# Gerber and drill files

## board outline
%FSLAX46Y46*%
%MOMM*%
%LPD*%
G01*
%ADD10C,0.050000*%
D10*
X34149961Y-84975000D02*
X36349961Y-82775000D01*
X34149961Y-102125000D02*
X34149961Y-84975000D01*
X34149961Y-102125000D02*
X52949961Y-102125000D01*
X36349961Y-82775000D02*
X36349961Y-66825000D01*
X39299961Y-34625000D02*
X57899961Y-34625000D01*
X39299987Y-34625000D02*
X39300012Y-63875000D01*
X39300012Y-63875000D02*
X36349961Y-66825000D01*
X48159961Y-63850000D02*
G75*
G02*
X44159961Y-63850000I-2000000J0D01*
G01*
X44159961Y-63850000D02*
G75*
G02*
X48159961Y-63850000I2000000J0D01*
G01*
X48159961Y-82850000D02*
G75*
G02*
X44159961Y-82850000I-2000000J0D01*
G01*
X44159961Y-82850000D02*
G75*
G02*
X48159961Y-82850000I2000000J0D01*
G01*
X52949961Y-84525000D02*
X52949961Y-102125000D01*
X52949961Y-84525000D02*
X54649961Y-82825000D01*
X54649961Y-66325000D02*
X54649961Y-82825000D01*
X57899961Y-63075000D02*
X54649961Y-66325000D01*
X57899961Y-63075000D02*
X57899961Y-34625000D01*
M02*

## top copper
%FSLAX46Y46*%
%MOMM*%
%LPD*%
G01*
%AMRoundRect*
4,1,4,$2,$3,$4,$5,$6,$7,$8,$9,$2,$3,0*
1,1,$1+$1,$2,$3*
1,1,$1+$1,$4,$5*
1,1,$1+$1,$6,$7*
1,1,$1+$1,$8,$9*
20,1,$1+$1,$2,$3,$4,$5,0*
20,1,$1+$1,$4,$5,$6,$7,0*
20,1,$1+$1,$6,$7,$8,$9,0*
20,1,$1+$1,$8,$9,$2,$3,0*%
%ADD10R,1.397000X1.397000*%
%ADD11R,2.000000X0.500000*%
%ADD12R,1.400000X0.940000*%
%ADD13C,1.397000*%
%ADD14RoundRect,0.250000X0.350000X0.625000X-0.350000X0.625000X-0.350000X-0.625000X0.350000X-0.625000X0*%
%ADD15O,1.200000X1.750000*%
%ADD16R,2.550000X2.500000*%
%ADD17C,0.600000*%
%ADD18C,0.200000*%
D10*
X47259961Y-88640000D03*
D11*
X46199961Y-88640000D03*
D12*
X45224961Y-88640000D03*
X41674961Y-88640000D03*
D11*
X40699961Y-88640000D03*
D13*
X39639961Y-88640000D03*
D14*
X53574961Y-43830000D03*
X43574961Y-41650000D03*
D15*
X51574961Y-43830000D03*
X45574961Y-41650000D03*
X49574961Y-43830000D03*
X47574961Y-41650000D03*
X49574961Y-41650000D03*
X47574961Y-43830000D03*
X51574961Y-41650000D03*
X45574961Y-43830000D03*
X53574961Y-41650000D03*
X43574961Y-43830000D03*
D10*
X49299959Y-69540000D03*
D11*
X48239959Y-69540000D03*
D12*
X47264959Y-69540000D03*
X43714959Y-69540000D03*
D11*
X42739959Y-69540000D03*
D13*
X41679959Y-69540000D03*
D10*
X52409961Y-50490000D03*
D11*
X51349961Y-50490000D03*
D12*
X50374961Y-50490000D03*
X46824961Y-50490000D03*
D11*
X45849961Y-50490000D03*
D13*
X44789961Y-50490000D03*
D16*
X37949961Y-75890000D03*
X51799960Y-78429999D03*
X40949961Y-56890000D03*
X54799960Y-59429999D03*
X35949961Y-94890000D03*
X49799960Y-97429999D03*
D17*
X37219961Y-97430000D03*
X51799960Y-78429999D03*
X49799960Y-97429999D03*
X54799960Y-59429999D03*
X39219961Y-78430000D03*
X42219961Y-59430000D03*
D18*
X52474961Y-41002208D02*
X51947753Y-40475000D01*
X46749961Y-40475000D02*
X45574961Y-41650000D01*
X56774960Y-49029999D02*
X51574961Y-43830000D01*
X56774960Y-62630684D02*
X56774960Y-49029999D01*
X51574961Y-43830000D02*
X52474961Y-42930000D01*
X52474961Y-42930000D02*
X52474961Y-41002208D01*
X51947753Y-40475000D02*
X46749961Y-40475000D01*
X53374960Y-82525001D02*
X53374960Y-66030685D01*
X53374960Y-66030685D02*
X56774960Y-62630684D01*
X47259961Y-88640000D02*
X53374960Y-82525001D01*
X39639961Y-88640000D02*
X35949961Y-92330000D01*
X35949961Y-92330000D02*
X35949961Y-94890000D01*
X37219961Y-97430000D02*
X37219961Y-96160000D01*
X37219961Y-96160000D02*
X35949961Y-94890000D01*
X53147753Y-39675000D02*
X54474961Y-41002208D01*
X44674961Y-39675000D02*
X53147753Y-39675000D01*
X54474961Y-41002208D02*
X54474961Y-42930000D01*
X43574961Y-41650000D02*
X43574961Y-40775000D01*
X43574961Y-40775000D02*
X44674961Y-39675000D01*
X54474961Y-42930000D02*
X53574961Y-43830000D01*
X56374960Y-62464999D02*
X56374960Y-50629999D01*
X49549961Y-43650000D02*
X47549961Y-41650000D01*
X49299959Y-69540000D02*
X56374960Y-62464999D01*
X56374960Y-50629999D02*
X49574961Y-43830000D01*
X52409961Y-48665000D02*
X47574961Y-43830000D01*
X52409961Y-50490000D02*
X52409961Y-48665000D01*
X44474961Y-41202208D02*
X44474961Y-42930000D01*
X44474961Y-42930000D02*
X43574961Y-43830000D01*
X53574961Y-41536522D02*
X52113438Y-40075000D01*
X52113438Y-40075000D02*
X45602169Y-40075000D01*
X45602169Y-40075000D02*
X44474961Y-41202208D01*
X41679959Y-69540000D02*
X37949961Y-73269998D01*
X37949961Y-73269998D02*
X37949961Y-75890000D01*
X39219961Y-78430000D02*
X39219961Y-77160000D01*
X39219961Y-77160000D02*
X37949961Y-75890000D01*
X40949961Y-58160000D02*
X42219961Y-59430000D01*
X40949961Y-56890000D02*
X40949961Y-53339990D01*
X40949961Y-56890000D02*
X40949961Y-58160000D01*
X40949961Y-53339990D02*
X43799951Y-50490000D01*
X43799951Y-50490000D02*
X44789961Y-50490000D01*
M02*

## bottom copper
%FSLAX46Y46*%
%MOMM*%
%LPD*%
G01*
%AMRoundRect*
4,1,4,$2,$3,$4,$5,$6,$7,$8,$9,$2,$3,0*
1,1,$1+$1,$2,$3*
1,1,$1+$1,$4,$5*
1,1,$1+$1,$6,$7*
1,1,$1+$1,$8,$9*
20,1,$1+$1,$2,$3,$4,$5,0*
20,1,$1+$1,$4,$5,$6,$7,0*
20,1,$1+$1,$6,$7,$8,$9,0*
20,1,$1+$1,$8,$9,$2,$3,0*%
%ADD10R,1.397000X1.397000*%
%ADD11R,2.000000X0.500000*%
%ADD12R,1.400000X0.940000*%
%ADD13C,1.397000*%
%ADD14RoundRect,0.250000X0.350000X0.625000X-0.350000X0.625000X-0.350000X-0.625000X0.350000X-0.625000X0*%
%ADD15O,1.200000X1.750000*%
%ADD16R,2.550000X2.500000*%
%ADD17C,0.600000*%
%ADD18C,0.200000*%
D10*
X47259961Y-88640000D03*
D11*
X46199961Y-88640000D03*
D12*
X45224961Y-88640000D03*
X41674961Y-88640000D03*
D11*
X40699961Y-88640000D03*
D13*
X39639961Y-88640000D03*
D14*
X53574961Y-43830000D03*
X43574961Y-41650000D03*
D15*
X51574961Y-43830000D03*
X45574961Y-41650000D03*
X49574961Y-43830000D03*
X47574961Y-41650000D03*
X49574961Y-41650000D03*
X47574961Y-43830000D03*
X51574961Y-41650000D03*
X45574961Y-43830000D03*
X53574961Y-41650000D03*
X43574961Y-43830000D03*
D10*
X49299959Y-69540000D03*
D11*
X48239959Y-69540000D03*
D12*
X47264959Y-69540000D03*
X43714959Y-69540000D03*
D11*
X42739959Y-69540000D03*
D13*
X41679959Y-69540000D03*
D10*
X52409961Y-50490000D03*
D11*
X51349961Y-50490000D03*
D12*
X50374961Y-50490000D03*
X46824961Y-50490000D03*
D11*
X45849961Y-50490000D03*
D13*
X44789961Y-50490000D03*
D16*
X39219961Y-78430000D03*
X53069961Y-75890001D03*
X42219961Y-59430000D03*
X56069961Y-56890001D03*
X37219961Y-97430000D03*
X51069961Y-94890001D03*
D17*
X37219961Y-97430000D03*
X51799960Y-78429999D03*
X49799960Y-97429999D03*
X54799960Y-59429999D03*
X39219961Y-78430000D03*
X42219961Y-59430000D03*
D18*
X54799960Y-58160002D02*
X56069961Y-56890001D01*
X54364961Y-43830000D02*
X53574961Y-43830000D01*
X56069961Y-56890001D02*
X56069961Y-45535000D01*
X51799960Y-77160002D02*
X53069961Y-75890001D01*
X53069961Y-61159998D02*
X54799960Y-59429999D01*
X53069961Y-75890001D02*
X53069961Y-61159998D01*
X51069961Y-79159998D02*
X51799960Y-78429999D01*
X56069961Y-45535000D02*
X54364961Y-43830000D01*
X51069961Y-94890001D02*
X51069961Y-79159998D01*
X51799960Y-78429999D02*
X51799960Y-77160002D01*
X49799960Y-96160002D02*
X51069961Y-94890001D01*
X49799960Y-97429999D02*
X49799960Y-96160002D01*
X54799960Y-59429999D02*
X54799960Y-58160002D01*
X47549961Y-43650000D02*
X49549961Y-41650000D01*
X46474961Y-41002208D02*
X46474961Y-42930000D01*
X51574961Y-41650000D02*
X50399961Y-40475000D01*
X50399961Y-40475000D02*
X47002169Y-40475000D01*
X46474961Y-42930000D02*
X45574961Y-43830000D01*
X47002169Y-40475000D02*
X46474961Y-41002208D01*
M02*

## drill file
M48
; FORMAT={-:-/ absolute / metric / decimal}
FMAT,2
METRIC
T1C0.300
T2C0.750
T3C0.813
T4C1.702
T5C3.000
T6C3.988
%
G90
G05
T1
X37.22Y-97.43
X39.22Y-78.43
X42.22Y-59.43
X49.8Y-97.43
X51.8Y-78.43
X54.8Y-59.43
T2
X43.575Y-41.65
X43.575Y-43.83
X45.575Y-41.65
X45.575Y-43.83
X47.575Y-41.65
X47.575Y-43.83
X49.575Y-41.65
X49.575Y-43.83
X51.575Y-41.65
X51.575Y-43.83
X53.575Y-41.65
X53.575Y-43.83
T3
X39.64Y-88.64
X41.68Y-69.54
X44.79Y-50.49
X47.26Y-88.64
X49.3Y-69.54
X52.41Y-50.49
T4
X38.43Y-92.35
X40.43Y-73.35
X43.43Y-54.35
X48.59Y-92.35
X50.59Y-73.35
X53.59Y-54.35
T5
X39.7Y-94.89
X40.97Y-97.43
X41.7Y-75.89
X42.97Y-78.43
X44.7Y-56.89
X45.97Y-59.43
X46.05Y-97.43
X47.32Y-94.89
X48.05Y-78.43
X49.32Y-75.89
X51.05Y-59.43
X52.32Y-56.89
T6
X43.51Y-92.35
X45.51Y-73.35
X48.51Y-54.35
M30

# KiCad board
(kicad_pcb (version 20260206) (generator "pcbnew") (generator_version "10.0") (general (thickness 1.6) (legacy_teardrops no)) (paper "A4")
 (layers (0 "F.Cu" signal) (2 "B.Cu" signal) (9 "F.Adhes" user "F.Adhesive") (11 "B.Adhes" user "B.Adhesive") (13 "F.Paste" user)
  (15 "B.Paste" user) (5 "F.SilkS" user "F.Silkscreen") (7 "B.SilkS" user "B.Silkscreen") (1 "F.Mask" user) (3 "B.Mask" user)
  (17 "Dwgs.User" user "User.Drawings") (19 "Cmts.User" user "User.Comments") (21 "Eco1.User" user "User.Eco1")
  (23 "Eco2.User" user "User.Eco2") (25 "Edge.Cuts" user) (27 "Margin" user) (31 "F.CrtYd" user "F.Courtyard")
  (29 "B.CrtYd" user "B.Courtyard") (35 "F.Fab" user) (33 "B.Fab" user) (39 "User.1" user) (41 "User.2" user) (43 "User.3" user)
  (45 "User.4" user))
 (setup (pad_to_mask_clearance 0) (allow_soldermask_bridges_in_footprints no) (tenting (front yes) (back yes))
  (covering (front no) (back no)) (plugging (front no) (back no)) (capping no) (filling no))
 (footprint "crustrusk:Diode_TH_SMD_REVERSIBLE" (layer "F.Cu") (at 43.449961 88.64 180)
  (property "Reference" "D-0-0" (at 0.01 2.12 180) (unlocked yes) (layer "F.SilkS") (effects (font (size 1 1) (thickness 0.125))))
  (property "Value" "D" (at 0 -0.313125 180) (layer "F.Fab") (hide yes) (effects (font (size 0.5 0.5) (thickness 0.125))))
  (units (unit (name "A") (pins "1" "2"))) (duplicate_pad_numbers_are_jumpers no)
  (pad "1" thru_hole rect (at -3.81 0 180) (size 1.397 1.397) (drill 0.8128) (layers "*.Cu" "*.Mask") (remove_unused_layers no)
   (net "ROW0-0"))
  (pad "1" smd rect (at -2.75 0) (size 2 0.5) (layers "F.Cu") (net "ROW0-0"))
  (pad "1" smd rect (at -2.75 0 180) (size 2 0.5) (layers "B.Cu") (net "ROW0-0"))
  (pad "1" smd rect (at -1.775 0) (size 1.4 0.94) (layers "F.Cu" "F.Mask" "F.Paste") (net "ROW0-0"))
  (pad "1" smd rect (at -1.775 0 180) (size 1.4 0.94) (layers "B.Cu" "B.Mask" "B.Paste") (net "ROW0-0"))
  (pad "2" smd rect (at 1.775 0) (size 1.4 0.94) (layers "F.Cu" "F.Mask" "F.Paste") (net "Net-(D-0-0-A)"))
  (pad "2" smd rect (at 1.775 0 180) (size 1.4 0.94) (layers "B.Cu" "B.Mask" "B.Paste") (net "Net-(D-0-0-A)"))
  (pad "2" smd rect (at 2.75 0) (size 2 0.5) (layers "F.Cu") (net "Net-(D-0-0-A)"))
  (pad "2" smd rect (at 2.75 0 180) (size 2 0.5) (layers "B.Cu") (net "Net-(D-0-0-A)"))
  (pad "2" thru_hole circle (at 3.81 0 180) (size 1.397 1.397) (drill 0.8128) (layers "*.Cu" "*.Mask") (remove_unused_layers no)
   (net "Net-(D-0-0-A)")))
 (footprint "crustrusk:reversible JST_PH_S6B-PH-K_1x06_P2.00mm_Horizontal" (layer "F.Cu") (at 53.574961 43.83 180)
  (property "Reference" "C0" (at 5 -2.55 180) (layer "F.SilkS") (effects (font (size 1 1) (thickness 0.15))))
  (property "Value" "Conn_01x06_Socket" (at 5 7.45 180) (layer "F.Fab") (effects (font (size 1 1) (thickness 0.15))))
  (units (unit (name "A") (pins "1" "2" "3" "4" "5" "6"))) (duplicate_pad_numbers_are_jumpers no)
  (pad "1" thru_hole roundrect (at 0 0 180) (size 1.2 1.75) (drill 0.75) (layers "*.Cu" "*.Mask") (remove_unused_layers no)
   (roundrect_rratio 0.208333) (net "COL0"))
  (pad "1" thru_hole roundrect (at 10 2.18 180) (size 1.2 1.75) (drill 0.75) (layers "*.Cu" "*.Mask") (remove_unused_layers no)
   (roundrect_rratio 0.208333) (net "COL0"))
  (pad "2" thru_hole oval (at 2 0 180) (size 1.2 1.75) (drill 0.75) (layers "*.Cu" "*.Mask") (remove_unused_layers no) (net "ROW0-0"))
  (pad "2" thru_hole oval (at 8 2.18 180) (size 1.2 1.75) (drill 0.75) (layers "*.Cu" "*.Mask") (remove_unused_layers no) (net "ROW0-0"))
  (pad "3" thru_hole oval (at 4 0 180) (size 1.2 1.75) (drill 0.75) (layers "*.Cu" "*.Mask") (remove_unused_layers no) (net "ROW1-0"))
  (pad "3" thru_hole oval (at 6 2.18 180) (size 1.2 1.75) (drill 0.75) (layers "*.Cu" "*.Mask") (remove_unused_layers no) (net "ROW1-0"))
  (pad "4" thru_hole oval (at 4 2.18 180) (size 1.2 1.75) (drill 0.75) (layers "*.Cu" "*.Mask") (remove_unused_layers no) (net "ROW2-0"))
  (pad "4" thru_hole oval (at 6 0 180) (size 1.2 1.75) (drill 0.75) (layers "*.Cu" "*.Mask") (remove_unused_layers no) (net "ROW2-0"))
  (pad "5" thru_hole oval (at 2 2.18 180) (size 1.2 1.75) (drill 0.75) (layers "*.Cu" "*.Mask") (remove_unused_layers no) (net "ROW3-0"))
  (pad "5" thru_hole oval (at 8 0 180) (size 1.2 1.75) (drill 0.75) (layers "*.Cu" "*.Mask") (remove_unused_layers no) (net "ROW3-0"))
  (pad "6" thru_hole oval (at 0 2.18 180) (size 1.2 1.75) (drill 0.75) (layers "*.Cu" "*.Mask") (remove_unused_layers no) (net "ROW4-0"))
  (pad "6" thru_hole oval (at 10 0 180) (size 1.2 1.75) (drill 0.75) (layers "*.Cu" "*.Mask") (remove_unused_layers no) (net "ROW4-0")))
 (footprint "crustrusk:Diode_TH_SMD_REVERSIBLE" (layer "F.Cu") (at 45.489959 69.54 180)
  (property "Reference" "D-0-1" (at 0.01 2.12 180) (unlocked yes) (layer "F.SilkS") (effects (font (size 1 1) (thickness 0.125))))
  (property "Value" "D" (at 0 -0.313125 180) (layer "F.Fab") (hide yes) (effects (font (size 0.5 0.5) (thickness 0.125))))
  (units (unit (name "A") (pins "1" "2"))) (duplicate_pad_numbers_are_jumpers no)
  (pad "1" thru_hole rect (at -3.81 0 180) (size 1.397 1.397) (drill 0.8128) (layers "*.Cu" "*.Mask") (remove_unused_layers no)
   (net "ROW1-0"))
  (pad "1" smd rect (at -2.75 0) (size 2 0.5) (layers "F.Cu") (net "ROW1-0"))
  (pad "1" smd rect (at -2.75 0 180) (size 2 0.5) (layers "B.Cu") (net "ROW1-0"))
  (pad "1" smd rect (at -1.775 0) (size 1.4 0.94) (layers "F.Cu" "F.Mask" "F.Paste") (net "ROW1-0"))
  (pad "1" smd rect (at -1.775 0 180) (size 1.4 0.94) (layers "B.Cu" "B.Mask" "B.Paste") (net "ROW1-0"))
  (pad "2" smd rect (at 1.775 0) (size 1.4 0.94) (layers "F.Cu" "F.Mask" "F.Paste") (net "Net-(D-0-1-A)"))
  (pad "2" smd rect (at 1.775 0 180) (size 1.4 0.94) (layers "B.Cu" "B.Mask" "B.Paste") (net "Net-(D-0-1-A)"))
  (pad "2" smd rect (at 2.75 0) (size 2 0.5) (layers "F.Cu") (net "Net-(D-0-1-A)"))
  (pad "2" smd rect (at 2.75 0 180) (size 2 0.5) (layers "B.Cu") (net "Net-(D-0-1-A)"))
  (pad "2" thru_hole circle (at 3.81 0 180) (size 1.397 1.397) (drill 0.8128) (layers "*.Cu" "*.Mask") (remove_unused_layers no)
   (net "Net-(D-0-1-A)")))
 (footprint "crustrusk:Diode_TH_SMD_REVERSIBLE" (layer "F.Cu") (at 48.599961 50.49 180)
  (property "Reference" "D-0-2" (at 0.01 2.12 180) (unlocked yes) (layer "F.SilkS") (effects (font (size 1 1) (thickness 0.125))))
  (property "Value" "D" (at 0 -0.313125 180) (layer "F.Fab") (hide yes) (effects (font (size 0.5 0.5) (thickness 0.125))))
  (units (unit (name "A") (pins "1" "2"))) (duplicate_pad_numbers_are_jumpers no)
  (pad "1" thru_hole rect (at -3.81 0 180) (size 1.397 1.397) (drill 0.8128) (layers "*.Cu" "*.Mask") (remove_unused_layers no)
   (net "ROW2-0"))
  (pad "1" smd rect (at -2.75 0) (size 2 0.5) (layers "F.Cu") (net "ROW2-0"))
  (pad "1" smd rect (at -2.75 0 180) (size 2 0.5) (layers "B.Cu") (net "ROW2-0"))
  (pad "1" smd rect (at -1.775 0) (size 1.4 0.94) (layers "F.Cu" "F.Mask" "F.Paste") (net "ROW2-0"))
  (pad "1" smd rect (at -1.775 0 180) (size 1.4 0.94) (layers "B.Cu" "B.Mask" "B.Paste") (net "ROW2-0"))
  (pad "2" smd rect (at 1.775 0) (size 1.4 0.94) (layers "F.Cu" "F.Mask" "F.Paste") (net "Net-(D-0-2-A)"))
  (pad "2" smd rect (at 1.775 0 180) (size 1.4 0.94) (layers "B.Cu" "B.Mask" "B.Paste") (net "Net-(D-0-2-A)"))
  (pad "2" smd rect (at 2.75 0) (size 2 0.5) (layers "F.Cu") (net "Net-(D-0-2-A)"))
  (pad "2" smd rect (at 2.75 0 180) (size 2 0.5) (layers "B.Cu") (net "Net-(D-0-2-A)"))
  (pad "2" thru_hole circle (at 3.81 0 180) (size 1.397 1.397) (drill 0.8128) (layers "*.Cu" "*.Mask") (remove_unused_layers no)
   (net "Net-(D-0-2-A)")))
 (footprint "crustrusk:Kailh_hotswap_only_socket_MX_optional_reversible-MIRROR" (layer "F.Cu") (at 45.509961 73.35 180)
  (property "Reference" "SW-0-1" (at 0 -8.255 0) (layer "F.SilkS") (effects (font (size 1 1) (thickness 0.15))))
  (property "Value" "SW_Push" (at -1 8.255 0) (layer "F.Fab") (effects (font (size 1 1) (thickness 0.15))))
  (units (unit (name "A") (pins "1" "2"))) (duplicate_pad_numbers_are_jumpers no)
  (pad "" np_thru_hole circle (at -5.08 0 180) (size 1.7018 1.7018) (drill 1.7018) (layers "*.Cu" "*.Mask"))
  (pad "" np_thru_hole circle (at -3.81 -2.54) (size 3 3) (drill 3) (layers "*.Cu" "*.Mask"))
  (pad "" np_thru_hole circle (at -2.54 -5.079998 180) (size 3 3) (drill 3) (layers "*.Cu" "*.Mask"))
  (pad "" np_thru_hole circle (at 0 0 180) (size 3.9878 3.9878) (drill 3.9878) (layers "*.Cu" "*.Mask"))
  (pad "" np_thru_hole circle (at 2.540002 -5.080001) (size 3 3) (drill 3) (layers "*.Cu" "*.Mask"))
  (pad "" np_thru_hole circle (at 3.81 -2.54 180) (size 3 3) (drill 3) (layers "*.Cu" "*.Mask"))
  (pad "" np_thru_hole circle (at 5.08 0 180) (size 1.7018 1.7018) (drill 1.7018) (layers "*.Cu" "*.Mask"))
  (pad "1" smd rect (at 6.29 -5.08) (size 2.55 2.5) (layers "B.Cu" "B.Mask" "B.Paste") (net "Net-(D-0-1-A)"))
  (pad "1" smd rect (at 7.56 -2.54 180) (size 2.55 2.5) (layers "F.Cu" "F.Mask" "F.Paste") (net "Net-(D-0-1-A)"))
  (pad "2" smd rect (at -7.56 -2.540001) (size 2.55 2.5) (layers "B.Cu" "B.Mask" "B.Paste") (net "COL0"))
  (pad "2" smd rect (at -6.289999 -5.079999 180) (size 2.55 2.5) (layers "F.Cu" "F.Mask" "F.Paste") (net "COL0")))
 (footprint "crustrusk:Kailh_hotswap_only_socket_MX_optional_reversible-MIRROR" (layer "F.Cu") (at 48.509961 54.35 180)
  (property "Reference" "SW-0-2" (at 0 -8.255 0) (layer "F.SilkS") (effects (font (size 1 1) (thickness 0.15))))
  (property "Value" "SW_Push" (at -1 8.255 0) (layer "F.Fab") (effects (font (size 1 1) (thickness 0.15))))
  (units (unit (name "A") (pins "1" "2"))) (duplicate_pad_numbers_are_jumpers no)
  (pad "" np_thru_hole circle (at -5.08 0 180) (size 1.7018 1.7018) (drill 1.7018) (layers "*.Cu" "*.Mask"))
  (pad "" np_thru_hole circle (at -3.81 -2.54) (size 3 3) (drill 3) (layers "*.Cu" "*.Mask"))
  (pad "" np_thru_hole circle (at -2.54 -5.079998 180) (size 3 3) (drill 3) (layers "*.Cu" "*.Mask"))
  (pad "" np_thru_hole circle (at 0 0 180) (size 3.9878 3.9878) (drill 3.9878) (layers "*.Cu" "*.Mask"))
  (pad "" np_thru_hole circle (at 2.540002 -5.080001) (size 3 3) (drill 3) (layers "*.Cu" "*.Mask"))
  (pad "" np_thru_hole circle (at 3.81 -2.54 180) (size 3 3) (drill 3) (layers "*.Cu" "*.Mask"))
  (pad "" np_thru_hole circle (at 5.08 0 180) (size 1.7018 1.7018) (drill 1.7018) (layers "*.Cu" "*.Mask"))
  (pad "1" smd rect (at 6.29 -5.08) (size 2.55 2.5) (layers "B.Cu" "B.Mask" "B.Paste") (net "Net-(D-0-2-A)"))
  (pad "1" smd rect (at 7.56 -2.54 180) (size 2.55 2.5) (layers "F.Cu" "F.Mask" "F.Paste") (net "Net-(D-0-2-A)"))
  (pad "2" smd rect (at -7.56 -2.540001) (size 2.55 2.5) (layers "B.Cu" "B.Mask" "B.Paste") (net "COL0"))
  (pad "2" smd rect (at -6.289999 -5.079999 180) (size 2.55 2.5) (layers "F.Cu" "F.Mask" "F.Paste") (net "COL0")))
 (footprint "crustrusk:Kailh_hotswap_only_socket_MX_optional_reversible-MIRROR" (layer "F.Cu") (at 43.509961 92.35 180)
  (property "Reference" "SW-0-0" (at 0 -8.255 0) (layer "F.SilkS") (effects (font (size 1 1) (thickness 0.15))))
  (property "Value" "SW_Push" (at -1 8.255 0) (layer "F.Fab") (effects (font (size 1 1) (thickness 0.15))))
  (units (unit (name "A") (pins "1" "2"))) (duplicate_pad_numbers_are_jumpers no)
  (pad "" np_thru_hole circle (at -5.08 0 180) (size 1.7018 1.7018) (drill 1.7018) (layers "*.Cu" "*.Mask"))
  (pad "" np_thru_hole circle (at -3.81 -2.54) (size 3 3) (drill 3) (layers "*.Cu" "*.Mask"))
  (pad "" np_thru_hole circle (at -2.54 -5.079998 180) (size 3 3) (drill 3) (layers "*.Cu" "*.Mask"))
  (pad "" np_thru_hole circle (at 0 0 180) (size 3.9878 3.9878) (drill 3.9878) (layers "*.Cu" "*.Mask"))
  (pad "" np_thru_hole circle (at 2.540002 -5.080001) (size 3 3) (drill 3) (layers "*.Cu" "*.Mask"))
  (pad "" np_thru_hole circle (at 3.81 -2.54 180) (size 3 3) (drill 3) (layers "*.Cu" "*.Mask"))
  (pad "" np_thru_hole circle (at 5.08 0 180) (size 1.7018 1.7018) (drill 1.7018) (layers "*.Cu" "*.Mask"))
  (pad "1" smd rect (at 6.29 -5.08) (size 2.55 2.5) (layers "B.Cu" "B.Mask" "B.Paste") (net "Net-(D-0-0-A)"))
  (pad "1" smd rect (at 7.56 -2.54 180) (size 2.55 2.5) (layers "F.Cu" "F.Mask" "F.Paste") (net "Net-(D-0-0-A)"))
  (pad "2" smd rect (at -7.56 -2.540001) (size 2.55 2.5) (layers "B.Cu" "B.Mask" "B.Paste") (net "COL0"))
  (pad "2" smd rect (at -6.289999 -5.079999 180) (size 2.55 2.5) (layers "F.Cu" "F.Mask" "F.Paste") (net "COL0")))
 (gr_line (start 34.149961 84.975) (end 36.349961 82.775) (stroke (width 0.05) (type default)) (layer "Edge.Cuts"))
 (gr_line (start 34.149961 102.125) (end 34.149961 84.975) (stroke (width 0.05) (type default)) (layer "Edge.Cuts"))
 (gr_line (start 34.149961 102.125) (end 52.949961 102.125) (stroke (width 0.05) (type default)) (layer "Edge.Cuts"))
 (gr_line (start 36.349961 82.775) (end 36.349961 66.825) (stroke (width 0.05) (type default)) (layer "Edge.Cuts"))
 (gr_line (start 39.299961 34.625) (end 57.899961 34.625) (stroke (width 0.05) (type default)) (layer "Edge.Cuts"))
 (gr_line (start 39.299987 34.625) (end 39.300012 63.875) (stroke (width 0.05) (type default)) (layer "Edge.Cuts"))
 (gr_line (start 39.300012 63.875) (end 36.349961 66.825) (stroke (width 0.05) (type default)) (layer "Edge.Cuts"))
 (gr_circle (center 46.159961 63.85) (end 46.159961 65.85) (stroke (width 0.05) (type default)) (fill no) (layer "Edge.Cuts"))
 (gr_circle (center 46.159961 82.85) (end 46.159961 84.85) (stroke (width 0.05) (type default)) (fill no) (layer "Edge.Cuts"))
 (gr_line (start 52.949961 84.525) (end 52.949961 102.125) (stroke (width 0.05) (type default)) (layer "Edge.Cuts"))
 (gr_line (start 52.949961 84.525) (end 54.649961 82.825) (stroke (width 0.05) (type default)) (layer "Edge.Cuts"))
 (gr_line (start 54.649961 66.325) (end 54.649961 82.825) (stroke (width 0.05) (type default)) (layer "Edge.Cuts"))
 (gr_line (start 57.899961 63.075) (end 54.649961 66.325) (stroke (width 0.05) (type default)) (layer "Edge.Cuts"))
 (gr_line (start 57.899961 63.075) (end 57.899961 34.625) (stroke (width 0.05) (type default)) (layer "Edge.Cuts"))
 (segment (start 52.474961 41.002208) (end 51.947753 40.475) (width 0.2) (layer "F.Cu") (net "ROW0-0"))
 (segment (start 46.749961 40.475) (end 45.574961 41.65) (width 0.2) (layer "F.Cu") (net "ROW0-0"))
 (segment (start 56.77496 49.029999) (end 51.574961 43.83) (width 0.2) (layer "F.Cu") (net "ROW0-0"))
 (segment (start 56.77496 62.630684) (end 56.77496 49.029999) (width 0.2) (layer "F.Cu") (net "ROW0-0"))
 (segment (start 51.574961 43.83) (end 52.474961 42.93) (width 0.2) (layer "F.Cu") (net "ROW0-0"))
 (segment (start 52.474961 42.93) (end 52.474961 41.002208) (width 0.2) (layer "F.Cu") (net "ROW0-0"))
 (segment (start 51.947753 40.475) (end 46.749961 40.475) (width 0.2) (layer "F.Cu") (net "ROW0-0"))
 (segment (start 53.37496 82.525001) (end 53.37496 66.030685) (width 0.2) (layer "F.Cu") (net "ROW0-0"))
 (segment (start 53.37496 66.030685) (end 56.77496 62.630684) (width 0.2) (layer "F.Cu") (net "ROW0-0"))
 (segment (start 47.259961 88.64) (end 53.37496 82.525001) (width 0.2) (layer "F.Cu") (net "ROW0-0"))
 (segment (start 39.639961 88.64) (end 35.949961 92.33) (width 0.2) (layer "F.Cu") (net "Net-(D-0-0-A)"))
 (segment (start 35.949961 92.33) (end 35.949961 94.89) (width 0.2) (layer "F.Cu") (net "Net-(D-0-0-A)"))
 (segment (start 37.219961 97.43) (end 37.219961 96.16) (width 0.2) (layer "F.Cu") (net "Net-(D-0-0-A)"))
 (segment (start 37.219961 96.16) (end 35.949961 94.89) (width 0.2) (layer "F.Cu") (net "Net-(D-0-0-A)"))
 (via (at 37.219961 97.43) (size 0.6) (drill 0.3) (layers "F.Cu" "B.Cu") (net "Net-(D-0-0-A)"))
 (segment (start 53.147753 39.675) (end 54.474961 41.002208) (width 0.2) (layer "F.Cu") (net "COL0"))
 (segment (start 44.674961 39.675) (end 53.147753 39.675) (width 0.2) (layer "F.Cu") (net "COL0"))
 (segment (start 54.474961 41.002208) (end 54.474961 42.93) (width 0.2) (layer "F.Cu") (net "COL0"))
 (segment (start 43.574961 41.65) (end 43.574961 40.775) (width 0.2) (layer "F.Cu") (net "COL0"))
 (segment (start 43.574961 40.775) (end 44.674961 39.675) (width 0.2) (layer "F.Cu") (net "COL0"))
 (segment (start 54.474961 42.93) (end 53.574961 43.83) (width 0.2) (layer "F.Cu") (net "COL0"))
 (via (at 51.79996 78.429999) (size 0.6) (drill 0.3) (layers "F.Cu" "B.Cu") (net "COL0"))
 (via (at 49.79996 97.429999) (size 0.6) (drill 0.3) (layers "F.Cu" "B.Cu") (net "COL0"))
 (via (at 54.79996 59.429999) (size 0.6) (drill 0.3) (layers "F.Cu" "B.Cu") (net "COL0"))
 (segment (start 54.79996 58.160002) (end 56.069961 56.890001) (width 0.2) (layer "B.Cu") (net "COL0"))
 (segment (start 54.364961 43.83) (end 53.574961 43.83) (width 0.2) (layer "B.Cu") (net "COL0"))
 (segment (start 56.069961 56.890001) (end 56.069961 45.535) (width 0.2) (layer "B.Cu") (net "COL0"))
 (segment (start 51.79996 77.160002) (end 53.069961 75.890001) (width 0.2) (layer "B.Cu") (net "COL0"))
 (segment (start 53.069961 61.159998) (end 54.79996 59.429999) (width 0.2) (layer "B.Cu") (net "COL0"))
 (segment (start 53.069961 75.890001) (end 53.069961 61.159998) (width 0.2) (layer "B.Cu") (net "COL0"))
 (segment (start 51.069961 79.159998) (end 51.79996 78.429999) (width 0.2) (layer "B.Cu") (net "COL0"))
 (segment (start 56.069961 45.535) (end 54.364961 43.83) (width 0.2) (layer "B.Cu") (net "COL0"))
 (segment (start 51.069961 94.890001) (end 51.069961 79.159998) (width 0.2) (layer "B.Cu") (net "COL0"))
 (segment (start 51.79996 78.429999) (end 51.79996 77.160002) (width 0.2) (layer "B.Cu") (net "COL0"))
 (segment (start 49.79996 96.160002) (end 51.069961 94.890001) (width 0.2) (layer "B.Cu") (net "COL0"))
 (segment (start 49.79996 97.429999) (end 49.79996 96.160002) (width 0.2) (layer "B.Cu") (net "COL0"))
 (segment (start 54.79996 59.429999) (end 54.79996 58.160002) (width 0.2) (layer "B.Cu") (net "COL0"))
 (segment (start 56.37496 62.464999) (end 56.37496 50.629999) (width 0.2) (layer "F.Cu") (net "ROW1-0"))
 (segment (start 49.549961 43.65) (end 47.549961 41.65) (width 0.2) (layer "F.Cu") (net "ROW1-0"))
 (segment (start 49.299959 69.54) (end 56.37496 62.464999) (width 0.2) (layer "F.Cu") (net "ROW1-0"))
 (segment (start 56.37496 50.629999) (end 49.574961 43.83) (width 0.2) (layer "F.Cu") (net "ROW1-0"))
 (segment (start 52.409961 48.665) (end 47.574961 43.83) (width 0.2) (layer "F.Cu") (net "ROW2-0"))
 (segment (start 52.409961 50.49) (end 52.409961 48.665) (width 0.2) (layer "F.Cu") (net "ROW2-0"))
 (segment (start 47.549961 43.65) (end 49.549961 41.65) (width 0.2) (layer "B.Cu") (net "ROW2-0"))
 (segment (start 46.474961 41.002208) (end 46.474961 42.93) (width 0.2) (layer "B.Cu") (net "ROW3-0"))
 (segment (start 51.574961 41.65) (end 50.399961 40.475) (width 0.2) (layer "B.Cu") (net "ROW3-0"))
 (segment (start 50.399961 40.475) (end 47.002169 40.475) (width 0.2) (layer "B.Cu") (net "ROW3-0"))
 (segment (start 46.474961 42.93) (end 45.574961 43.83) (width 0.2) (layer "B.Cu") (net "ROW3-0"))
 (segment (start 47.002169 40.475) (end 46.474961 41.002208) (width 0.2) (layer "B.Cu") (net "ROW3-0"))
 (segment (start 44.474961 41.202208) (end 44.474961 42.93) (width 0.2) (layer "F.Cu") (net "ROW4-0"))
 (segment (start 44.474961 42.93) (end 43.574961 43.83) (width 0.2) (layer "F.Cu") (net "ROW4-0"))
 (segment (start 53.574961 41.536522) (end 52.113438 40.075) (width 0.2) (layer "F.Cu") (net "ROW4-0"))
 (segment (start 52.113438 40.075) (end 45.602169 40.075) (width 0.2) (layer "F.Cu") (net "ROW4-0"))
 (segment (start 45.602169 40.075) (end 44.474961 41.202208) (width 0.2) (layer "F.Cu") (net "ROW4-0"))
 (segment (start 41.679959 69.54) (end 37.949961 73.269998) (width 0.2) (layer "F.Cu") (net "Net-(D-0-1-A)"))
 (segment (start 37.949961 73.269998) (end 37.949961 75.89) (width 0.2) (layer "F.Cu") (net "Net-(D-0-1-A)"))
 (segment (start 39.219961 78.43) (end 39.219961 77.16) (width 0.2) (layer "F.Cu") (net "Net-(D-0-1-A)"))
 (segment (start 39.219961 77.16) (end 37.949961 75.89) (width 0.2) (layer "F.Cu") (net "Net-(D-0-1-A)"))
 (via (at 39.219961 78.43) (size 0.6) (drill 0.3) (layers "F.Cu" "B.Cu") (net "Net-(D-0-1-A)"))
 (segment (start 40.949961 58.16) (end 42.219961 59.43) (width 0.2) (layer "F.Cu") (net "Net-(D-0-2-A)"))
 (segment (start 40.949961 56.89) (end 40.949961 53.33999) (width 0.2) (layer "F.Cu") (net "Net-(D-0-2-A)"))
 (segment (start 40.949961 56.89) (end 40.949961 58.16) (width 0.2) (layer "F.Cu") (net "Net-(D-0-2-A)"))
 (segment (start 40.949961 53.33999) (end 43.799951 50.49) (width 0.2) (layer "F.Cu") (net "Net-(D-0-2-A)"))
 (segment (start 43.799951 50.49) (end 44.789961 50.49) (width 0.2) (layer "F.Cu") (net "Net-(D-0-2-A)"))
 (via (at 42.219961 59.43) (size 0.6) (drill 0.3) (layers "F.Cu" "B.Cu") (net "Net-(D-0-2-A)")))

